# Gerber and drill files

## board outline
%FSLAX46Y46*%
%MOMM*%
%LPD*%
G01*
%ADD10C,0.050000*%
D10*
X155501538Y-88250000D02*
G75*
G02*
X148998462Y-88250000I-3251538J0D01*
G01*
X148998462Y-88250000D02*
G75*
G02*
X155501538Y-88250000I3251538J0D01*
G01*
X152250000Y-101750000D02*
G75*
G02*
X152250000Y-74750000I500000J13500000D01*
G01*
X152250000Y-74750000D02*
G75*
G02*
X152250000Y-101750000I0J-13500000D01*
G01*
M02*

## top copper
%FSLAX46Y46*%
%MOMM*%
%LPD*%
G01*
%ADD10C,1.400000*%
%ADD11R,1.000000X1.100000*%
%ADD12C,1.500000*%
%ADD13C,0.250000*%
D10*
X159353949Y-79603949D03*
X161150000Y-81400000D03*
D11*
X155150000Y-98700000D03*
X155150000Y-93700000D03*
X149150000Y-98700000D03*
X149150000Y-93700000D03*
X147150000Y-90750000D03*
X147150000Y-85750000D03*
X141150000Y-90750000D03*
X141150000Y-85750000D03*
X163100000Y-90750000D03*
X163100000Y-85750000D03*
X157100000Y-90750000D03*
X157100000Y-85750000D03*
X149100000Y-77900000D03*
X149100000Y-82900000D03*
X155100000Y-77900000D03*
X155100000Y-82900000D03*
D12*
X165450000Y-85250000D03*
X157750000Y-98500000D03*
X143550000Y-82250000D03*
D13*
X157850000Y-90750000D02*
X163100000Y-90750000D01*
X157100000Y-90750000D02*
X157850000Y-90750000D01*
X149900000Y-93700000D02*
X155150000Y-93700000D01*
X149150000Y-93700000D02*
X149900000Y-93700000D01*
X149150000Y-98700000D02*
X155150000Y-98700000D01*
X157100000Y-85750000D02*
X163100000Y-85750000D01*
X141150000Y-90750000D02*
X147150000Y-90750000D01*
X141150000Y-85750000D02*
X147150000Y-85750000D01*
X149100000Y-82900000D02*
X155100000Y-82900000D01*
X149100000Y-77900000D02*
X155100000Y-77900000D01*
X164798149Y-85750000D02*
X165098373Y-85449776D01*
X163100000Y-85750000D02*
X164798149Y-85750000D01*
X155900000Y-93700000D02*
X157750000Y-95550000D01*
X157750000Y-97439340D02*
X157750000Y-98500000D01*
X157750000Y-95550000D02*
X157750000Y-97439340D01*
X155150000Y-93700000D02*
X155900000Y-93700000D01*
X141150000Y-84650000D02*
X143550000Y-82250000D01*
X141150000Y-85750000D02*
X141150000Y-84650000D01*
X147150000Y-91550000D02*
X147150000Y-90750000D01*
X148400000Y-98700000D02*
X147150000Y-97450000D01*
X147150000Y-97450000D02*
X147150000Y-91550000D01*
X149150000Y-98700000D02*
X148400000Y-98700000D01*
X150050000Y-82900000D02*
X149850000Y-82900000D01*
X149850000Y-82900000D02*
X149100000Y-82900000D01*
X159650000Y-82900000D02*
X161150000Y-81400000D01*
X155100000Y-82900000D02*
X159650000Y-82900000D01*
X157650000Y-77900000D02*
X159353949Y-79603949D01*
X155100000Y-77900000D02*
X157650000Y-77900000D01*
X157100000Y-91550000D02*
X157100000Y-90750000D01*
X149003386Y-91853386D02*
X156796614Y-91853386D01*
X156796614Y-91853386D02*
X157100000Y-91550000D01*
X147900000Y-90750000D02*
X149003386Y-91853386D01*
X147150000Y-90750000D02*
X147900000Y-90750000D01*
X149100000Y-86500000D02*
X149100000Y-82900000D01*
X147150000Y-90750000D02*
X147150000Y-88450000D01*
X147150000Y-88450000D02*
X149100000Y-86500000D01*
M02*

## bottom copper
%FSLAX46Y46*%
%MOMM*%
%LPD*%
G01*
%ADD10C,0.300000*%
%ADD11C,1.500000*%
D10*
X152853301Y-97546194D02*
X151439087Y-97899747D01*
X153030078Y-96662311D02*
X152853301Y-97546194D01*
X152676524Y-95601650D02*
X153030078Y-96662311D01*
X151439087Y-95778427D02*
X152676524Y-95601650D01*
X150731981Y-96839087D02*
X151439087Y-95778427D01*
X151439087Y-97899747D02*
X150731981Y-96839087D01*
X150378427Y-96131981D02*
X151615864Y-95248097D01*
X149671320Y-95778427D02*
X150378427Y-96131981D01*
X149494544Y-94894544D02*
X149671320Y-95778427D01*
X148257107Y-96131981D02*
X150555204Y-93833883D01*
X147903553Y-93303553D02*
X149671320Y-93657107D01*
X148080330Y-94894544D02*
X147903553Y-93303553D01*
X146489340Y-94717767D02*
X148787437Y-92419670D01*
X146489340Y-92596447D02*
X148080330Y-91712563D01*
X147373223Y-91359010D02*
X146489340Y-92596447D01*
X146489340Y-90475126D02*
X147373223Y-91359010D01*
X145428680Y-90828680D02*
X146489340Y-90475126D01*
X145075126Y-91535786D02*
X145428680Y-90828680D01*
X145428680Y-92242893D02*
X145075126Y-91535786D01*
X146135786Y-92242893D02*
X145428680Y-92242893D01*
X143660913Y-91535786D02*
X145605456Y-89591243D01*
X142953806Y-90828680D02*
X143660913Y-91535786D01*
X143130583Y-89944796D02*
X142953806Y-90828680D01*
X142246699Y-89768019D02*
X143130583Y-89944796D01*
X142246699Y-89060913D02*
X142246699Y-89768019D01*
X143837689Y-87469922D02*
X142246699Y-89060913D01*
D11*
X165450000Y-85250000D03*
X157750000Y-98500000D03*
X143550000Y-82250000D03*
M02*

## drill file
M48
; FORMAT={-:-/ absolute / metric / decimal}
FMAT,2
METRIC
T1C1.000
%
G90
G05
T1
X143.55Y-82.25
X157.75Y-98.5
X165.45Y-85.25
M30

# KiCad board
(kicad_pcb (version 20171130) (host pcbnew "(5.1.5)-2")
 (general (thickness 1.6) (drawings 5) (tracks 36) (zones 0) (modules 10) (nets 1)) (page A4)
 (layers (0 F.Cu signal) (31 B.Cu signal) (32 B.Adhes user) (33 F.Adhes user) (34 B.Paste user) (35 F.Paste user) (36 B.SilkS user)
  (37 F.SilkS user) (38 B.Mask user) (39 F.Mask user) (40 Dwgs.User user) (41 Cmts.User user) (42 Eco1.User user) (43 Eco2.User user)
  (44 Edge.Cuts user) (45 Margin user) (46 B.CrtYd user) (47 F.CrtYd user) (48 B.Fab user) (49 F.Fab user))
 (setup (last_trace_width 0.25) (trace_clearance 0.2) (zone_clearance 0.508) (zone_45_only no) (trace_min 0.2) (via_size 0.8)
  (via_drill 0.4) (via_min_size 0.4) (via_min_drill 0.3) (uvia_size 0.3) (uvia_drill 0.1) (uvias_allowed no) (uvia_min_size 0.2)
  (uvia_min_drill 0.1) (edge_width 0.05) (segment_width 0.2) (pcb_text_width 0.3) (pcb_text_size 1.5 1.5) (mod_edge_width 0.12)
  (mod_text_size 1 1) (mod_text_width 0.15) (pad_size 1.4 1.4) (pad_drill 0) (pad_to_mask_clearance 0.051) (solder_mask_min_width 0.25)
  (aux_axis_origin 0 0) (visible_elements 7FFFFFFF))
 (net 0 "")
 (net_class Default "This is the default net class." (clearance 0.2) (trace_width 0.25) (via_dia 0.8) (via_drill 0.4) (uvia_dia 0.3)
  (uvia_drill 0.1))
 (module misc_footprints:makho (layer B.Cu) (at 147.55 92.95 315)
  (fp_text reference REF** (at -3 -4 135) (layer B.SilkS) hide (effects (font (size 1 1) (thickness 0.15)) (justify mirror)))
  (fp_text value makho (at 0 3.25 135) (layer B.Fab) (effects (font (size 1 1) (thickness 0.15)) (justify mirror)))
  (fp_line (start 7 -0.5) (end 6.25 0.75) (layer B.Cu) (width 0.3))
  (fp_line (start 6.5 -1.25) (end 7 -0.5) (layer B.Cu) (width 0.3))
  (fp_line (start 5.5 -1.75) (end 6.5 -1.25) (layer B.Cu) (width 0.3))
  (fp_line (start 4.75 -0.75) (end 5.5 -1.75) (layer B.Cu) (width 0.3))
  (fp_line (start 5 0.5) (end 4.75 -0.75) (layer B.Cu) (width 0.3))
  (fp_line (start 6.25 0.75) (end 5 0.5) (layer B.Cu) (width 0.3))
  (fp_line (start 4.25 0.25) (end 4.5 -1.25) (layer B.Cu) (width 0.3))
  (fp_line (start 3.5 0.5) (end 4.25 0.25) (layer B.Cu) (width 0.3))
  (fp_line (start 2.75 0) (end 3.5 0.5) (layer B.Cu) (width 0.3))
  (fp_line (start 2.75 1.75) (end 2.75 -1.5) (layer B.Cu) (width 0.3)) (fp_line (start 0.5 0) (end 2 -1) (layer B.Cu) (width 0.3))
  (fp_line (start 1.75 1) (end 0.5 0) (layer B.Cu) (width 0.3))
  (fp_line (start 0.5 2) (end 0.5 -1.25) (layer B.Cu) (width 0.3))
  (fp_line (start -1 0.5) (end -0.5 -1.25) (layer B.Cu) (width 0.3))
  (fp_line (start -1.25 -1) (end -1 0.5) (layer B.Cu) (width 0.3))
  (fp_line (start -2.5 -1) (end -1.25 -1) (layer B.Cu) (width 0.3))
  (fp_line (start -3 0) (end -2.5 -1) (layer B.Cu) (width 0.3))
  (fp_line (start -2.75 0.75) (end -3 0) (layer B.Cu) (width 0.3))
  (fp_line (start -2 1) (end -2.75 0.75) (layer B.Cu) (width 0.3))
  (fp_line (start -1.5 0.5) (end -2 1) (layer B.Cu) (width 0.3))
  (fp_line (start -3.75 1.75) (end -3.75 -1) (layer B.Cu) (width 0.3))
  (fp_line (start -4.75 1.75) (end -3.75 1.75) (layer B.Cu) (width 0.3))
  (fp_line (start -5.25 1) (end -4.75 1.75) (layer B.Cu) (width 0.3))
  (fp_line (start -6 1.5) (end -5.25 1) (layer B.Cu) (width 0.3))
  (fp_line (start -6.5 1) (end -6 1.5) (layer B.Cu) (width 0.3))
  (fp_line (start -6.5 -1.25) (end -6.5 1) (layer B.Cu) (width 0.3)))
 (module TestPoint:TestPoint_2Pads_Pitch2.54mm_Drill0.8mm (layer F.Cu) (at 161.15 81.4 135)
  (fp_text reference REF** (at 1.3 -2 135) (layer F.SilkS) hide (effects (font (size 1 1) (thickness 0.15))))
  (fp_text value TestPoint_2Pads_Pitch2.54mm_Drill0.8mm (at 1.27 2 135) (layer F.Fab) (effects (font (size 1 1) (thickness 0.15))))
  (pad 2 smd circle (at 2.54 0 135) (size 1.4 1.4) (layers F.Cu F.Paste F.Mask))
  (pad 1 smd circle (at 0 0 135) (size 1.4 1.4) (layers F.Cu F.Paste F.Mask)))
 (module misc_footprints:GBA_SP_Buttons (layer F.Cu) (at 152.15 96.2)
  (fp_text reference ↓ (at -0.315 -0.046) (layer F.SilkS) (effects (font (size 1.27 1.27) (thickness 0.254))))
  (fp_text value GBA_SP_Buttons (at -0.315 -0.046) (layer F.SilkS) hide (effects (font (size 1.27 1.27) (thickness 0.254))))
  (pad 4 smd rect (at 3 2.5) (size 1 1.1) (layers F.Cu F.Paste F.Mask))
  (pad 3 smd rect (at 3 -2.5) (size 1 1.1) (layers F.Cu F.Paste F.Mask))
  (pad 2 smd rect (at -3 2.5) (size 1 1.1) (layers F.Cu F.Paste F.Mask))
  (pad 1 smd rect (at -3 -2.5) (size 1 1.1) (layers F.Cu F.Paste F.Mask)))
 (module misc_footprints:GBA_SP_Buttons (layer F.Cu) (at 144.15 88.25)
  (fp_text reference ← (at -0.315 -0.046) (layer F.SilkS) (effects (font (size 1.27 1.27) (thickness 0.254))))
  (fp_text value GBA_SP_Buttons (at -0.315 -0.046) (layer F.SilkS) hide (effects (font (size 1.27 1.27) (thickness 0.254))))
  (pad 4 smd rect (at 3 2.5) (size 1 1.1) (layers F.Cu F.Paste F.Mask))
  (pad 3 smd rect (at 3 -2.5) (size 1 1.1) (layers F.Cu F.Paste F.Mask))
  (pad 2 smd rect (at -3 2.5) (size 1 1.1) (layers F.Cu F.Paste F.Mask))
  (pad 1 smd rect (at -3 -2.5) (size 1 1.1) (layers F.Cu F.Paste F.Mask)))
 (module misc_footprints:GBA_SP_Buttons (layer F.Cu) (at 160.1 88.25)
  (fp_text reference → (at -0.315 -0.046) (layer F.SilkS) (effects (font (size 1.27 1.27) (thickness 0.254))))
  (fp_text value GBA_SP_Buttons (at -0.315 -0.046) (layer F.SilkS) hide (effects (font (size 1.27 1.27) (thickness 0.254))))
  (pad 4 smd rect (at 3 2.5) (size 1 1.1) (layers F.Cu F.Paste F.Mask))
  (pad 3 smd rect (at 3 -2.5) (size 1 1.1) (layers F.Cu F.Paste F.Mask))
  (pad 2 smd rect (at -3 2.5) (size 1 1.1) (layers F.Cu F.Paste F.Mask))
  (pad 1 smd rect (at -3 -2.5) (size 1 1.1) (layers F.Cu F.Paste F.Mask)))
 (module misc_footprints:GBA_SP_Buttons (layer F.Cu) (at 152.1 80.4)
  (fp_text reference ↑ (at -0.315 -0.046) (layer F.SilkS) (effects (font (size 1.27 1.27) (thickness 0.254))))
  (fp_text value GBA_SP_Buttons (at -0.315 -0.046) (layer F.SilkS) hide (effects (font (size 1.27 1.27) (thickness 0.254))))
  (pad 1 smd rect (at -3 -2.5) (size 1 1.1) (layers F.Cu F.Paste F.Mask))
  (pad 2 smd rect (at -3 2.5) (size 1 1.1) (layers F.Cu F.Paste F.Mask))
  (pad 3 smd rect (at 3 -2.5) (size 1 1.1) (layers F.Cu F.Paste F.Mask))
  (pad 4 smd rect (at 3 2.5) (size 1 1.1) (layers F.Cu F.Paste F.Mask)))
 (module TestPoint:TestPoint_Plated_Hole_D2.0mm (layer F.Cu) (at 165.45 85.25)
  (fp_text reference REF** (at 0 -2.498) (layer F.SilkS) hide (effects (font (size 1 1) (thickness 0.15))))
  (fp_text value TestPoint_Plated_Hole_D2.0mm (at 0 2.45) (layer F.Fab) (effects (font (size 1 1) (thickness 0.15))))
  (pad 1 thru_hole circle (at 0 0) (size 1.5 1.5) (drill 1) (layers *.Cu *.Mask)))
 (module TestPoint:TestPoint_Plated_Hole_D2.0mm (layer F.Cu) (at 157.75 98.5)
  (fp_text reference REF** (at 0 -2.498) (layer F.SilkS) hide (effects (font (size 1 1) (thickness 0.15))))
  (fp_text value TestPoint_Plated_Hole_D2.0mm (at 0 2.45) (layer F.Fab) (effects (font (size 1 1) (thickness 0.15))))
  (pad 1 thru_hole circle (at 0 0) (size 1.5 1.5) (drill 1) (layers *.Cu *.Mask)))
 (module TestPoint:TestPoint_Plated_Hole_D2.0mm (layer F.Cu) (at 143.55 82.25)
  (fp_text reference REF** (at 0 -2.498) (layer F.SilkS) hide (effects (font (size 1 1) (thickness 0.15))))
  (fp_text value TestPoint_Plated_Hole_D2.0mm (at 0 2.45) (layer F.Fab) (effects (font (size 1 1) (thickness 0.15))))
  (pad 1 thru_hole circle (at 0 0) (size 1.5 1.5) (drill 1) (layers *.Cu *.Mask)))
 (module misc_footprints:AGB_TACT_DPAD (layer F.Cu) (at 152.225 88.275)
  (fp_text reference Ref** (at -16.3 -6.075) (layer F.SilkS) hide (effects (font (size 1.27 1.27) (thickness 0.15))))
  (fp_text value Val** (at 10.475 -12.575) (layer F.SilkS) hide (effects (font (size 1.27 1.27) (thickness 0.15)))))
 (gr_circle (center 152.25 88.25) (end 155.5 88.35) (layer Edge.Cuts) (width 0.05))
 (gr_arc (start 152.75 88.25) (end 152.25 74.75) (angle -175.7578072) (layer Edge.Cuts) (width 0.05))
 (gr_arc (start 152.25 88.25) (end 152.25 101.75) (angle -180) (layer Edge.Cuts) (width 0.05))
 (segment (start 157.85 90.75) (end 163.1 90.75) (width 0.25) (layer F.Cu) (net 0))
 (segment (start 157.1 90.75) (end 157.85 90.75) (width 0.25) (layer F.Cu) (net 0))
 (segment (start 149.9 93.7) (end 155.15 93.7) (width 0.25) (layer F.Cu) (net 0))
 (segment (start 149.15 93.7) (end 149.9 93.7) (width 0.25) (layer F.Cu) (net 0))
 (segment (start 149.15 98.7) (end 155.15 98.7) (width 0.25) (layer F.Cu) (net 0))
 (segment (start 157.1 85.75) (end 163.1 85.75) (width 0.25) (layer F.Cu) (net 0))
 (segment (start 141.15 90.75) (end 147.15 90.75) (width 0.25) (layer F.Cu) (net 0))
 (segment (start 141.15 85.75) (end 147.15 85.75) (width 0.25) (layer F.Cu) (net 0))
 (segment (start 149.1 82.9) (end 155.1 82.9) (width 0.25) (layer F.Cu) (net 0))
 (segment (start 149.1 77.9) (end 155.1 77.9) (width 0.25) (layer F.Cu) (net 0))
 (segment (start 164.798149 85.75) (end 165.098373 85.449776) (width 0.25) (layer F.Cu) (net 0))
 (segment (start 163.1 85.75) (end 164.798149 85.75) (width 0.25) (layer F.Cu) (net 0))
 (segment (start 155.9 93.7) (end 157.75 95.55) (width 0.25) (layer F.Cu) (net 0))
 (segment (start 157.75 97.43934) (end 157.75 98.5) (width 0.25) (layer F.Cu) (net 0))
 (segment (start 157.75 95.55) (end 157.75 97.43934) (width 0.25) (layer F.Cu) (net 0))
 (segment (start 155.15 93.7) (end 155.9 93.7) (width 0.25) (layer F.Cu) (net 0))
 (segment (start 141.15 84.65) (end 143.55 82.25) (width 0.25) (layer F.Cu) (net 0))
 (segment (start 141.15 85.75) (end 141.15 84.65) (width 0.25) (layer F.Cu) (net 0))
 (segment (start 147.15 91.55) (end 147.15 90.75) (width 0.25) (layer F.Cu) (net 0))
 (segment (start 148.4 98.7) (end 147.15 97.45) (width 0.25) (layer F.Cu) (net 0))
 (segment (start 147.15 97.45) (end 147.15 91.55) (width 0.25) (layer F.Cu) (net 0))
 (segment (start 149.15 98.7) (end 148.4 98.7) (width 0.25) (layer F.Cu) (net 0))
 (segment (start 150.05 82.9) (end 149.85 82.9) (width 0.25) (layer F.Cu) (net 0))
 (segment (start 149.85 82.9) (end 149.1 82.9) (width 0.25) (layer F.Cu) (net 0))
 (segment (start 159.65 82.9) (end 161.15 81.4) (width 0.25) (layer F.Cu) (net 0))
 (segment (start 155.1 82.9) (end 159.65 82.9) (width 0.25) (layer F.Cu) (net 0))
 (segment (start 157.65 77.9) (end 159.353949 79.603949) (width 0.25) (layer F.Cu) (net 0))
 (segment (start 155.1 77.9) (end 157.65 77.9) (width 0.25) (layer F.Cu) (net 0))
 (segment (start 157.1 91.55) (end 157.1 90.75) (width 0.25) (layer F.Cu) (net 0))
 (segment (start 149.003386 91.853386) (end 156.796614 91.853386) (width 0.25) (layer F.Cu) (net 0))
 (segment (start 156.796614 91.853386) (end 157.1 91.55) (width 0.25) (layer F.Cu) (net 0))
 (segment (start 147.9 90.75) (end 149.003386 91.853386) (width 0.25) (layer F.Cu) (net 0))
 (segment (start 147.15 90.75) (end 147.9 90.75) (width 0.25) (layer F.Cu) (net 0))
 (segment (start 149.1 86.5) (end 149.1 82.9) (width 0.25) (layer F.Cu) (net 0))
 (segment (start 147.15 90.75) (end 147.15 88.45) (width 0.25) (layer F.Cu) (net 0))
 (segment (start 147.15 88.45) (end 149.1 86.5) (width 0.25) (layer F.Cu) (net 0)))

